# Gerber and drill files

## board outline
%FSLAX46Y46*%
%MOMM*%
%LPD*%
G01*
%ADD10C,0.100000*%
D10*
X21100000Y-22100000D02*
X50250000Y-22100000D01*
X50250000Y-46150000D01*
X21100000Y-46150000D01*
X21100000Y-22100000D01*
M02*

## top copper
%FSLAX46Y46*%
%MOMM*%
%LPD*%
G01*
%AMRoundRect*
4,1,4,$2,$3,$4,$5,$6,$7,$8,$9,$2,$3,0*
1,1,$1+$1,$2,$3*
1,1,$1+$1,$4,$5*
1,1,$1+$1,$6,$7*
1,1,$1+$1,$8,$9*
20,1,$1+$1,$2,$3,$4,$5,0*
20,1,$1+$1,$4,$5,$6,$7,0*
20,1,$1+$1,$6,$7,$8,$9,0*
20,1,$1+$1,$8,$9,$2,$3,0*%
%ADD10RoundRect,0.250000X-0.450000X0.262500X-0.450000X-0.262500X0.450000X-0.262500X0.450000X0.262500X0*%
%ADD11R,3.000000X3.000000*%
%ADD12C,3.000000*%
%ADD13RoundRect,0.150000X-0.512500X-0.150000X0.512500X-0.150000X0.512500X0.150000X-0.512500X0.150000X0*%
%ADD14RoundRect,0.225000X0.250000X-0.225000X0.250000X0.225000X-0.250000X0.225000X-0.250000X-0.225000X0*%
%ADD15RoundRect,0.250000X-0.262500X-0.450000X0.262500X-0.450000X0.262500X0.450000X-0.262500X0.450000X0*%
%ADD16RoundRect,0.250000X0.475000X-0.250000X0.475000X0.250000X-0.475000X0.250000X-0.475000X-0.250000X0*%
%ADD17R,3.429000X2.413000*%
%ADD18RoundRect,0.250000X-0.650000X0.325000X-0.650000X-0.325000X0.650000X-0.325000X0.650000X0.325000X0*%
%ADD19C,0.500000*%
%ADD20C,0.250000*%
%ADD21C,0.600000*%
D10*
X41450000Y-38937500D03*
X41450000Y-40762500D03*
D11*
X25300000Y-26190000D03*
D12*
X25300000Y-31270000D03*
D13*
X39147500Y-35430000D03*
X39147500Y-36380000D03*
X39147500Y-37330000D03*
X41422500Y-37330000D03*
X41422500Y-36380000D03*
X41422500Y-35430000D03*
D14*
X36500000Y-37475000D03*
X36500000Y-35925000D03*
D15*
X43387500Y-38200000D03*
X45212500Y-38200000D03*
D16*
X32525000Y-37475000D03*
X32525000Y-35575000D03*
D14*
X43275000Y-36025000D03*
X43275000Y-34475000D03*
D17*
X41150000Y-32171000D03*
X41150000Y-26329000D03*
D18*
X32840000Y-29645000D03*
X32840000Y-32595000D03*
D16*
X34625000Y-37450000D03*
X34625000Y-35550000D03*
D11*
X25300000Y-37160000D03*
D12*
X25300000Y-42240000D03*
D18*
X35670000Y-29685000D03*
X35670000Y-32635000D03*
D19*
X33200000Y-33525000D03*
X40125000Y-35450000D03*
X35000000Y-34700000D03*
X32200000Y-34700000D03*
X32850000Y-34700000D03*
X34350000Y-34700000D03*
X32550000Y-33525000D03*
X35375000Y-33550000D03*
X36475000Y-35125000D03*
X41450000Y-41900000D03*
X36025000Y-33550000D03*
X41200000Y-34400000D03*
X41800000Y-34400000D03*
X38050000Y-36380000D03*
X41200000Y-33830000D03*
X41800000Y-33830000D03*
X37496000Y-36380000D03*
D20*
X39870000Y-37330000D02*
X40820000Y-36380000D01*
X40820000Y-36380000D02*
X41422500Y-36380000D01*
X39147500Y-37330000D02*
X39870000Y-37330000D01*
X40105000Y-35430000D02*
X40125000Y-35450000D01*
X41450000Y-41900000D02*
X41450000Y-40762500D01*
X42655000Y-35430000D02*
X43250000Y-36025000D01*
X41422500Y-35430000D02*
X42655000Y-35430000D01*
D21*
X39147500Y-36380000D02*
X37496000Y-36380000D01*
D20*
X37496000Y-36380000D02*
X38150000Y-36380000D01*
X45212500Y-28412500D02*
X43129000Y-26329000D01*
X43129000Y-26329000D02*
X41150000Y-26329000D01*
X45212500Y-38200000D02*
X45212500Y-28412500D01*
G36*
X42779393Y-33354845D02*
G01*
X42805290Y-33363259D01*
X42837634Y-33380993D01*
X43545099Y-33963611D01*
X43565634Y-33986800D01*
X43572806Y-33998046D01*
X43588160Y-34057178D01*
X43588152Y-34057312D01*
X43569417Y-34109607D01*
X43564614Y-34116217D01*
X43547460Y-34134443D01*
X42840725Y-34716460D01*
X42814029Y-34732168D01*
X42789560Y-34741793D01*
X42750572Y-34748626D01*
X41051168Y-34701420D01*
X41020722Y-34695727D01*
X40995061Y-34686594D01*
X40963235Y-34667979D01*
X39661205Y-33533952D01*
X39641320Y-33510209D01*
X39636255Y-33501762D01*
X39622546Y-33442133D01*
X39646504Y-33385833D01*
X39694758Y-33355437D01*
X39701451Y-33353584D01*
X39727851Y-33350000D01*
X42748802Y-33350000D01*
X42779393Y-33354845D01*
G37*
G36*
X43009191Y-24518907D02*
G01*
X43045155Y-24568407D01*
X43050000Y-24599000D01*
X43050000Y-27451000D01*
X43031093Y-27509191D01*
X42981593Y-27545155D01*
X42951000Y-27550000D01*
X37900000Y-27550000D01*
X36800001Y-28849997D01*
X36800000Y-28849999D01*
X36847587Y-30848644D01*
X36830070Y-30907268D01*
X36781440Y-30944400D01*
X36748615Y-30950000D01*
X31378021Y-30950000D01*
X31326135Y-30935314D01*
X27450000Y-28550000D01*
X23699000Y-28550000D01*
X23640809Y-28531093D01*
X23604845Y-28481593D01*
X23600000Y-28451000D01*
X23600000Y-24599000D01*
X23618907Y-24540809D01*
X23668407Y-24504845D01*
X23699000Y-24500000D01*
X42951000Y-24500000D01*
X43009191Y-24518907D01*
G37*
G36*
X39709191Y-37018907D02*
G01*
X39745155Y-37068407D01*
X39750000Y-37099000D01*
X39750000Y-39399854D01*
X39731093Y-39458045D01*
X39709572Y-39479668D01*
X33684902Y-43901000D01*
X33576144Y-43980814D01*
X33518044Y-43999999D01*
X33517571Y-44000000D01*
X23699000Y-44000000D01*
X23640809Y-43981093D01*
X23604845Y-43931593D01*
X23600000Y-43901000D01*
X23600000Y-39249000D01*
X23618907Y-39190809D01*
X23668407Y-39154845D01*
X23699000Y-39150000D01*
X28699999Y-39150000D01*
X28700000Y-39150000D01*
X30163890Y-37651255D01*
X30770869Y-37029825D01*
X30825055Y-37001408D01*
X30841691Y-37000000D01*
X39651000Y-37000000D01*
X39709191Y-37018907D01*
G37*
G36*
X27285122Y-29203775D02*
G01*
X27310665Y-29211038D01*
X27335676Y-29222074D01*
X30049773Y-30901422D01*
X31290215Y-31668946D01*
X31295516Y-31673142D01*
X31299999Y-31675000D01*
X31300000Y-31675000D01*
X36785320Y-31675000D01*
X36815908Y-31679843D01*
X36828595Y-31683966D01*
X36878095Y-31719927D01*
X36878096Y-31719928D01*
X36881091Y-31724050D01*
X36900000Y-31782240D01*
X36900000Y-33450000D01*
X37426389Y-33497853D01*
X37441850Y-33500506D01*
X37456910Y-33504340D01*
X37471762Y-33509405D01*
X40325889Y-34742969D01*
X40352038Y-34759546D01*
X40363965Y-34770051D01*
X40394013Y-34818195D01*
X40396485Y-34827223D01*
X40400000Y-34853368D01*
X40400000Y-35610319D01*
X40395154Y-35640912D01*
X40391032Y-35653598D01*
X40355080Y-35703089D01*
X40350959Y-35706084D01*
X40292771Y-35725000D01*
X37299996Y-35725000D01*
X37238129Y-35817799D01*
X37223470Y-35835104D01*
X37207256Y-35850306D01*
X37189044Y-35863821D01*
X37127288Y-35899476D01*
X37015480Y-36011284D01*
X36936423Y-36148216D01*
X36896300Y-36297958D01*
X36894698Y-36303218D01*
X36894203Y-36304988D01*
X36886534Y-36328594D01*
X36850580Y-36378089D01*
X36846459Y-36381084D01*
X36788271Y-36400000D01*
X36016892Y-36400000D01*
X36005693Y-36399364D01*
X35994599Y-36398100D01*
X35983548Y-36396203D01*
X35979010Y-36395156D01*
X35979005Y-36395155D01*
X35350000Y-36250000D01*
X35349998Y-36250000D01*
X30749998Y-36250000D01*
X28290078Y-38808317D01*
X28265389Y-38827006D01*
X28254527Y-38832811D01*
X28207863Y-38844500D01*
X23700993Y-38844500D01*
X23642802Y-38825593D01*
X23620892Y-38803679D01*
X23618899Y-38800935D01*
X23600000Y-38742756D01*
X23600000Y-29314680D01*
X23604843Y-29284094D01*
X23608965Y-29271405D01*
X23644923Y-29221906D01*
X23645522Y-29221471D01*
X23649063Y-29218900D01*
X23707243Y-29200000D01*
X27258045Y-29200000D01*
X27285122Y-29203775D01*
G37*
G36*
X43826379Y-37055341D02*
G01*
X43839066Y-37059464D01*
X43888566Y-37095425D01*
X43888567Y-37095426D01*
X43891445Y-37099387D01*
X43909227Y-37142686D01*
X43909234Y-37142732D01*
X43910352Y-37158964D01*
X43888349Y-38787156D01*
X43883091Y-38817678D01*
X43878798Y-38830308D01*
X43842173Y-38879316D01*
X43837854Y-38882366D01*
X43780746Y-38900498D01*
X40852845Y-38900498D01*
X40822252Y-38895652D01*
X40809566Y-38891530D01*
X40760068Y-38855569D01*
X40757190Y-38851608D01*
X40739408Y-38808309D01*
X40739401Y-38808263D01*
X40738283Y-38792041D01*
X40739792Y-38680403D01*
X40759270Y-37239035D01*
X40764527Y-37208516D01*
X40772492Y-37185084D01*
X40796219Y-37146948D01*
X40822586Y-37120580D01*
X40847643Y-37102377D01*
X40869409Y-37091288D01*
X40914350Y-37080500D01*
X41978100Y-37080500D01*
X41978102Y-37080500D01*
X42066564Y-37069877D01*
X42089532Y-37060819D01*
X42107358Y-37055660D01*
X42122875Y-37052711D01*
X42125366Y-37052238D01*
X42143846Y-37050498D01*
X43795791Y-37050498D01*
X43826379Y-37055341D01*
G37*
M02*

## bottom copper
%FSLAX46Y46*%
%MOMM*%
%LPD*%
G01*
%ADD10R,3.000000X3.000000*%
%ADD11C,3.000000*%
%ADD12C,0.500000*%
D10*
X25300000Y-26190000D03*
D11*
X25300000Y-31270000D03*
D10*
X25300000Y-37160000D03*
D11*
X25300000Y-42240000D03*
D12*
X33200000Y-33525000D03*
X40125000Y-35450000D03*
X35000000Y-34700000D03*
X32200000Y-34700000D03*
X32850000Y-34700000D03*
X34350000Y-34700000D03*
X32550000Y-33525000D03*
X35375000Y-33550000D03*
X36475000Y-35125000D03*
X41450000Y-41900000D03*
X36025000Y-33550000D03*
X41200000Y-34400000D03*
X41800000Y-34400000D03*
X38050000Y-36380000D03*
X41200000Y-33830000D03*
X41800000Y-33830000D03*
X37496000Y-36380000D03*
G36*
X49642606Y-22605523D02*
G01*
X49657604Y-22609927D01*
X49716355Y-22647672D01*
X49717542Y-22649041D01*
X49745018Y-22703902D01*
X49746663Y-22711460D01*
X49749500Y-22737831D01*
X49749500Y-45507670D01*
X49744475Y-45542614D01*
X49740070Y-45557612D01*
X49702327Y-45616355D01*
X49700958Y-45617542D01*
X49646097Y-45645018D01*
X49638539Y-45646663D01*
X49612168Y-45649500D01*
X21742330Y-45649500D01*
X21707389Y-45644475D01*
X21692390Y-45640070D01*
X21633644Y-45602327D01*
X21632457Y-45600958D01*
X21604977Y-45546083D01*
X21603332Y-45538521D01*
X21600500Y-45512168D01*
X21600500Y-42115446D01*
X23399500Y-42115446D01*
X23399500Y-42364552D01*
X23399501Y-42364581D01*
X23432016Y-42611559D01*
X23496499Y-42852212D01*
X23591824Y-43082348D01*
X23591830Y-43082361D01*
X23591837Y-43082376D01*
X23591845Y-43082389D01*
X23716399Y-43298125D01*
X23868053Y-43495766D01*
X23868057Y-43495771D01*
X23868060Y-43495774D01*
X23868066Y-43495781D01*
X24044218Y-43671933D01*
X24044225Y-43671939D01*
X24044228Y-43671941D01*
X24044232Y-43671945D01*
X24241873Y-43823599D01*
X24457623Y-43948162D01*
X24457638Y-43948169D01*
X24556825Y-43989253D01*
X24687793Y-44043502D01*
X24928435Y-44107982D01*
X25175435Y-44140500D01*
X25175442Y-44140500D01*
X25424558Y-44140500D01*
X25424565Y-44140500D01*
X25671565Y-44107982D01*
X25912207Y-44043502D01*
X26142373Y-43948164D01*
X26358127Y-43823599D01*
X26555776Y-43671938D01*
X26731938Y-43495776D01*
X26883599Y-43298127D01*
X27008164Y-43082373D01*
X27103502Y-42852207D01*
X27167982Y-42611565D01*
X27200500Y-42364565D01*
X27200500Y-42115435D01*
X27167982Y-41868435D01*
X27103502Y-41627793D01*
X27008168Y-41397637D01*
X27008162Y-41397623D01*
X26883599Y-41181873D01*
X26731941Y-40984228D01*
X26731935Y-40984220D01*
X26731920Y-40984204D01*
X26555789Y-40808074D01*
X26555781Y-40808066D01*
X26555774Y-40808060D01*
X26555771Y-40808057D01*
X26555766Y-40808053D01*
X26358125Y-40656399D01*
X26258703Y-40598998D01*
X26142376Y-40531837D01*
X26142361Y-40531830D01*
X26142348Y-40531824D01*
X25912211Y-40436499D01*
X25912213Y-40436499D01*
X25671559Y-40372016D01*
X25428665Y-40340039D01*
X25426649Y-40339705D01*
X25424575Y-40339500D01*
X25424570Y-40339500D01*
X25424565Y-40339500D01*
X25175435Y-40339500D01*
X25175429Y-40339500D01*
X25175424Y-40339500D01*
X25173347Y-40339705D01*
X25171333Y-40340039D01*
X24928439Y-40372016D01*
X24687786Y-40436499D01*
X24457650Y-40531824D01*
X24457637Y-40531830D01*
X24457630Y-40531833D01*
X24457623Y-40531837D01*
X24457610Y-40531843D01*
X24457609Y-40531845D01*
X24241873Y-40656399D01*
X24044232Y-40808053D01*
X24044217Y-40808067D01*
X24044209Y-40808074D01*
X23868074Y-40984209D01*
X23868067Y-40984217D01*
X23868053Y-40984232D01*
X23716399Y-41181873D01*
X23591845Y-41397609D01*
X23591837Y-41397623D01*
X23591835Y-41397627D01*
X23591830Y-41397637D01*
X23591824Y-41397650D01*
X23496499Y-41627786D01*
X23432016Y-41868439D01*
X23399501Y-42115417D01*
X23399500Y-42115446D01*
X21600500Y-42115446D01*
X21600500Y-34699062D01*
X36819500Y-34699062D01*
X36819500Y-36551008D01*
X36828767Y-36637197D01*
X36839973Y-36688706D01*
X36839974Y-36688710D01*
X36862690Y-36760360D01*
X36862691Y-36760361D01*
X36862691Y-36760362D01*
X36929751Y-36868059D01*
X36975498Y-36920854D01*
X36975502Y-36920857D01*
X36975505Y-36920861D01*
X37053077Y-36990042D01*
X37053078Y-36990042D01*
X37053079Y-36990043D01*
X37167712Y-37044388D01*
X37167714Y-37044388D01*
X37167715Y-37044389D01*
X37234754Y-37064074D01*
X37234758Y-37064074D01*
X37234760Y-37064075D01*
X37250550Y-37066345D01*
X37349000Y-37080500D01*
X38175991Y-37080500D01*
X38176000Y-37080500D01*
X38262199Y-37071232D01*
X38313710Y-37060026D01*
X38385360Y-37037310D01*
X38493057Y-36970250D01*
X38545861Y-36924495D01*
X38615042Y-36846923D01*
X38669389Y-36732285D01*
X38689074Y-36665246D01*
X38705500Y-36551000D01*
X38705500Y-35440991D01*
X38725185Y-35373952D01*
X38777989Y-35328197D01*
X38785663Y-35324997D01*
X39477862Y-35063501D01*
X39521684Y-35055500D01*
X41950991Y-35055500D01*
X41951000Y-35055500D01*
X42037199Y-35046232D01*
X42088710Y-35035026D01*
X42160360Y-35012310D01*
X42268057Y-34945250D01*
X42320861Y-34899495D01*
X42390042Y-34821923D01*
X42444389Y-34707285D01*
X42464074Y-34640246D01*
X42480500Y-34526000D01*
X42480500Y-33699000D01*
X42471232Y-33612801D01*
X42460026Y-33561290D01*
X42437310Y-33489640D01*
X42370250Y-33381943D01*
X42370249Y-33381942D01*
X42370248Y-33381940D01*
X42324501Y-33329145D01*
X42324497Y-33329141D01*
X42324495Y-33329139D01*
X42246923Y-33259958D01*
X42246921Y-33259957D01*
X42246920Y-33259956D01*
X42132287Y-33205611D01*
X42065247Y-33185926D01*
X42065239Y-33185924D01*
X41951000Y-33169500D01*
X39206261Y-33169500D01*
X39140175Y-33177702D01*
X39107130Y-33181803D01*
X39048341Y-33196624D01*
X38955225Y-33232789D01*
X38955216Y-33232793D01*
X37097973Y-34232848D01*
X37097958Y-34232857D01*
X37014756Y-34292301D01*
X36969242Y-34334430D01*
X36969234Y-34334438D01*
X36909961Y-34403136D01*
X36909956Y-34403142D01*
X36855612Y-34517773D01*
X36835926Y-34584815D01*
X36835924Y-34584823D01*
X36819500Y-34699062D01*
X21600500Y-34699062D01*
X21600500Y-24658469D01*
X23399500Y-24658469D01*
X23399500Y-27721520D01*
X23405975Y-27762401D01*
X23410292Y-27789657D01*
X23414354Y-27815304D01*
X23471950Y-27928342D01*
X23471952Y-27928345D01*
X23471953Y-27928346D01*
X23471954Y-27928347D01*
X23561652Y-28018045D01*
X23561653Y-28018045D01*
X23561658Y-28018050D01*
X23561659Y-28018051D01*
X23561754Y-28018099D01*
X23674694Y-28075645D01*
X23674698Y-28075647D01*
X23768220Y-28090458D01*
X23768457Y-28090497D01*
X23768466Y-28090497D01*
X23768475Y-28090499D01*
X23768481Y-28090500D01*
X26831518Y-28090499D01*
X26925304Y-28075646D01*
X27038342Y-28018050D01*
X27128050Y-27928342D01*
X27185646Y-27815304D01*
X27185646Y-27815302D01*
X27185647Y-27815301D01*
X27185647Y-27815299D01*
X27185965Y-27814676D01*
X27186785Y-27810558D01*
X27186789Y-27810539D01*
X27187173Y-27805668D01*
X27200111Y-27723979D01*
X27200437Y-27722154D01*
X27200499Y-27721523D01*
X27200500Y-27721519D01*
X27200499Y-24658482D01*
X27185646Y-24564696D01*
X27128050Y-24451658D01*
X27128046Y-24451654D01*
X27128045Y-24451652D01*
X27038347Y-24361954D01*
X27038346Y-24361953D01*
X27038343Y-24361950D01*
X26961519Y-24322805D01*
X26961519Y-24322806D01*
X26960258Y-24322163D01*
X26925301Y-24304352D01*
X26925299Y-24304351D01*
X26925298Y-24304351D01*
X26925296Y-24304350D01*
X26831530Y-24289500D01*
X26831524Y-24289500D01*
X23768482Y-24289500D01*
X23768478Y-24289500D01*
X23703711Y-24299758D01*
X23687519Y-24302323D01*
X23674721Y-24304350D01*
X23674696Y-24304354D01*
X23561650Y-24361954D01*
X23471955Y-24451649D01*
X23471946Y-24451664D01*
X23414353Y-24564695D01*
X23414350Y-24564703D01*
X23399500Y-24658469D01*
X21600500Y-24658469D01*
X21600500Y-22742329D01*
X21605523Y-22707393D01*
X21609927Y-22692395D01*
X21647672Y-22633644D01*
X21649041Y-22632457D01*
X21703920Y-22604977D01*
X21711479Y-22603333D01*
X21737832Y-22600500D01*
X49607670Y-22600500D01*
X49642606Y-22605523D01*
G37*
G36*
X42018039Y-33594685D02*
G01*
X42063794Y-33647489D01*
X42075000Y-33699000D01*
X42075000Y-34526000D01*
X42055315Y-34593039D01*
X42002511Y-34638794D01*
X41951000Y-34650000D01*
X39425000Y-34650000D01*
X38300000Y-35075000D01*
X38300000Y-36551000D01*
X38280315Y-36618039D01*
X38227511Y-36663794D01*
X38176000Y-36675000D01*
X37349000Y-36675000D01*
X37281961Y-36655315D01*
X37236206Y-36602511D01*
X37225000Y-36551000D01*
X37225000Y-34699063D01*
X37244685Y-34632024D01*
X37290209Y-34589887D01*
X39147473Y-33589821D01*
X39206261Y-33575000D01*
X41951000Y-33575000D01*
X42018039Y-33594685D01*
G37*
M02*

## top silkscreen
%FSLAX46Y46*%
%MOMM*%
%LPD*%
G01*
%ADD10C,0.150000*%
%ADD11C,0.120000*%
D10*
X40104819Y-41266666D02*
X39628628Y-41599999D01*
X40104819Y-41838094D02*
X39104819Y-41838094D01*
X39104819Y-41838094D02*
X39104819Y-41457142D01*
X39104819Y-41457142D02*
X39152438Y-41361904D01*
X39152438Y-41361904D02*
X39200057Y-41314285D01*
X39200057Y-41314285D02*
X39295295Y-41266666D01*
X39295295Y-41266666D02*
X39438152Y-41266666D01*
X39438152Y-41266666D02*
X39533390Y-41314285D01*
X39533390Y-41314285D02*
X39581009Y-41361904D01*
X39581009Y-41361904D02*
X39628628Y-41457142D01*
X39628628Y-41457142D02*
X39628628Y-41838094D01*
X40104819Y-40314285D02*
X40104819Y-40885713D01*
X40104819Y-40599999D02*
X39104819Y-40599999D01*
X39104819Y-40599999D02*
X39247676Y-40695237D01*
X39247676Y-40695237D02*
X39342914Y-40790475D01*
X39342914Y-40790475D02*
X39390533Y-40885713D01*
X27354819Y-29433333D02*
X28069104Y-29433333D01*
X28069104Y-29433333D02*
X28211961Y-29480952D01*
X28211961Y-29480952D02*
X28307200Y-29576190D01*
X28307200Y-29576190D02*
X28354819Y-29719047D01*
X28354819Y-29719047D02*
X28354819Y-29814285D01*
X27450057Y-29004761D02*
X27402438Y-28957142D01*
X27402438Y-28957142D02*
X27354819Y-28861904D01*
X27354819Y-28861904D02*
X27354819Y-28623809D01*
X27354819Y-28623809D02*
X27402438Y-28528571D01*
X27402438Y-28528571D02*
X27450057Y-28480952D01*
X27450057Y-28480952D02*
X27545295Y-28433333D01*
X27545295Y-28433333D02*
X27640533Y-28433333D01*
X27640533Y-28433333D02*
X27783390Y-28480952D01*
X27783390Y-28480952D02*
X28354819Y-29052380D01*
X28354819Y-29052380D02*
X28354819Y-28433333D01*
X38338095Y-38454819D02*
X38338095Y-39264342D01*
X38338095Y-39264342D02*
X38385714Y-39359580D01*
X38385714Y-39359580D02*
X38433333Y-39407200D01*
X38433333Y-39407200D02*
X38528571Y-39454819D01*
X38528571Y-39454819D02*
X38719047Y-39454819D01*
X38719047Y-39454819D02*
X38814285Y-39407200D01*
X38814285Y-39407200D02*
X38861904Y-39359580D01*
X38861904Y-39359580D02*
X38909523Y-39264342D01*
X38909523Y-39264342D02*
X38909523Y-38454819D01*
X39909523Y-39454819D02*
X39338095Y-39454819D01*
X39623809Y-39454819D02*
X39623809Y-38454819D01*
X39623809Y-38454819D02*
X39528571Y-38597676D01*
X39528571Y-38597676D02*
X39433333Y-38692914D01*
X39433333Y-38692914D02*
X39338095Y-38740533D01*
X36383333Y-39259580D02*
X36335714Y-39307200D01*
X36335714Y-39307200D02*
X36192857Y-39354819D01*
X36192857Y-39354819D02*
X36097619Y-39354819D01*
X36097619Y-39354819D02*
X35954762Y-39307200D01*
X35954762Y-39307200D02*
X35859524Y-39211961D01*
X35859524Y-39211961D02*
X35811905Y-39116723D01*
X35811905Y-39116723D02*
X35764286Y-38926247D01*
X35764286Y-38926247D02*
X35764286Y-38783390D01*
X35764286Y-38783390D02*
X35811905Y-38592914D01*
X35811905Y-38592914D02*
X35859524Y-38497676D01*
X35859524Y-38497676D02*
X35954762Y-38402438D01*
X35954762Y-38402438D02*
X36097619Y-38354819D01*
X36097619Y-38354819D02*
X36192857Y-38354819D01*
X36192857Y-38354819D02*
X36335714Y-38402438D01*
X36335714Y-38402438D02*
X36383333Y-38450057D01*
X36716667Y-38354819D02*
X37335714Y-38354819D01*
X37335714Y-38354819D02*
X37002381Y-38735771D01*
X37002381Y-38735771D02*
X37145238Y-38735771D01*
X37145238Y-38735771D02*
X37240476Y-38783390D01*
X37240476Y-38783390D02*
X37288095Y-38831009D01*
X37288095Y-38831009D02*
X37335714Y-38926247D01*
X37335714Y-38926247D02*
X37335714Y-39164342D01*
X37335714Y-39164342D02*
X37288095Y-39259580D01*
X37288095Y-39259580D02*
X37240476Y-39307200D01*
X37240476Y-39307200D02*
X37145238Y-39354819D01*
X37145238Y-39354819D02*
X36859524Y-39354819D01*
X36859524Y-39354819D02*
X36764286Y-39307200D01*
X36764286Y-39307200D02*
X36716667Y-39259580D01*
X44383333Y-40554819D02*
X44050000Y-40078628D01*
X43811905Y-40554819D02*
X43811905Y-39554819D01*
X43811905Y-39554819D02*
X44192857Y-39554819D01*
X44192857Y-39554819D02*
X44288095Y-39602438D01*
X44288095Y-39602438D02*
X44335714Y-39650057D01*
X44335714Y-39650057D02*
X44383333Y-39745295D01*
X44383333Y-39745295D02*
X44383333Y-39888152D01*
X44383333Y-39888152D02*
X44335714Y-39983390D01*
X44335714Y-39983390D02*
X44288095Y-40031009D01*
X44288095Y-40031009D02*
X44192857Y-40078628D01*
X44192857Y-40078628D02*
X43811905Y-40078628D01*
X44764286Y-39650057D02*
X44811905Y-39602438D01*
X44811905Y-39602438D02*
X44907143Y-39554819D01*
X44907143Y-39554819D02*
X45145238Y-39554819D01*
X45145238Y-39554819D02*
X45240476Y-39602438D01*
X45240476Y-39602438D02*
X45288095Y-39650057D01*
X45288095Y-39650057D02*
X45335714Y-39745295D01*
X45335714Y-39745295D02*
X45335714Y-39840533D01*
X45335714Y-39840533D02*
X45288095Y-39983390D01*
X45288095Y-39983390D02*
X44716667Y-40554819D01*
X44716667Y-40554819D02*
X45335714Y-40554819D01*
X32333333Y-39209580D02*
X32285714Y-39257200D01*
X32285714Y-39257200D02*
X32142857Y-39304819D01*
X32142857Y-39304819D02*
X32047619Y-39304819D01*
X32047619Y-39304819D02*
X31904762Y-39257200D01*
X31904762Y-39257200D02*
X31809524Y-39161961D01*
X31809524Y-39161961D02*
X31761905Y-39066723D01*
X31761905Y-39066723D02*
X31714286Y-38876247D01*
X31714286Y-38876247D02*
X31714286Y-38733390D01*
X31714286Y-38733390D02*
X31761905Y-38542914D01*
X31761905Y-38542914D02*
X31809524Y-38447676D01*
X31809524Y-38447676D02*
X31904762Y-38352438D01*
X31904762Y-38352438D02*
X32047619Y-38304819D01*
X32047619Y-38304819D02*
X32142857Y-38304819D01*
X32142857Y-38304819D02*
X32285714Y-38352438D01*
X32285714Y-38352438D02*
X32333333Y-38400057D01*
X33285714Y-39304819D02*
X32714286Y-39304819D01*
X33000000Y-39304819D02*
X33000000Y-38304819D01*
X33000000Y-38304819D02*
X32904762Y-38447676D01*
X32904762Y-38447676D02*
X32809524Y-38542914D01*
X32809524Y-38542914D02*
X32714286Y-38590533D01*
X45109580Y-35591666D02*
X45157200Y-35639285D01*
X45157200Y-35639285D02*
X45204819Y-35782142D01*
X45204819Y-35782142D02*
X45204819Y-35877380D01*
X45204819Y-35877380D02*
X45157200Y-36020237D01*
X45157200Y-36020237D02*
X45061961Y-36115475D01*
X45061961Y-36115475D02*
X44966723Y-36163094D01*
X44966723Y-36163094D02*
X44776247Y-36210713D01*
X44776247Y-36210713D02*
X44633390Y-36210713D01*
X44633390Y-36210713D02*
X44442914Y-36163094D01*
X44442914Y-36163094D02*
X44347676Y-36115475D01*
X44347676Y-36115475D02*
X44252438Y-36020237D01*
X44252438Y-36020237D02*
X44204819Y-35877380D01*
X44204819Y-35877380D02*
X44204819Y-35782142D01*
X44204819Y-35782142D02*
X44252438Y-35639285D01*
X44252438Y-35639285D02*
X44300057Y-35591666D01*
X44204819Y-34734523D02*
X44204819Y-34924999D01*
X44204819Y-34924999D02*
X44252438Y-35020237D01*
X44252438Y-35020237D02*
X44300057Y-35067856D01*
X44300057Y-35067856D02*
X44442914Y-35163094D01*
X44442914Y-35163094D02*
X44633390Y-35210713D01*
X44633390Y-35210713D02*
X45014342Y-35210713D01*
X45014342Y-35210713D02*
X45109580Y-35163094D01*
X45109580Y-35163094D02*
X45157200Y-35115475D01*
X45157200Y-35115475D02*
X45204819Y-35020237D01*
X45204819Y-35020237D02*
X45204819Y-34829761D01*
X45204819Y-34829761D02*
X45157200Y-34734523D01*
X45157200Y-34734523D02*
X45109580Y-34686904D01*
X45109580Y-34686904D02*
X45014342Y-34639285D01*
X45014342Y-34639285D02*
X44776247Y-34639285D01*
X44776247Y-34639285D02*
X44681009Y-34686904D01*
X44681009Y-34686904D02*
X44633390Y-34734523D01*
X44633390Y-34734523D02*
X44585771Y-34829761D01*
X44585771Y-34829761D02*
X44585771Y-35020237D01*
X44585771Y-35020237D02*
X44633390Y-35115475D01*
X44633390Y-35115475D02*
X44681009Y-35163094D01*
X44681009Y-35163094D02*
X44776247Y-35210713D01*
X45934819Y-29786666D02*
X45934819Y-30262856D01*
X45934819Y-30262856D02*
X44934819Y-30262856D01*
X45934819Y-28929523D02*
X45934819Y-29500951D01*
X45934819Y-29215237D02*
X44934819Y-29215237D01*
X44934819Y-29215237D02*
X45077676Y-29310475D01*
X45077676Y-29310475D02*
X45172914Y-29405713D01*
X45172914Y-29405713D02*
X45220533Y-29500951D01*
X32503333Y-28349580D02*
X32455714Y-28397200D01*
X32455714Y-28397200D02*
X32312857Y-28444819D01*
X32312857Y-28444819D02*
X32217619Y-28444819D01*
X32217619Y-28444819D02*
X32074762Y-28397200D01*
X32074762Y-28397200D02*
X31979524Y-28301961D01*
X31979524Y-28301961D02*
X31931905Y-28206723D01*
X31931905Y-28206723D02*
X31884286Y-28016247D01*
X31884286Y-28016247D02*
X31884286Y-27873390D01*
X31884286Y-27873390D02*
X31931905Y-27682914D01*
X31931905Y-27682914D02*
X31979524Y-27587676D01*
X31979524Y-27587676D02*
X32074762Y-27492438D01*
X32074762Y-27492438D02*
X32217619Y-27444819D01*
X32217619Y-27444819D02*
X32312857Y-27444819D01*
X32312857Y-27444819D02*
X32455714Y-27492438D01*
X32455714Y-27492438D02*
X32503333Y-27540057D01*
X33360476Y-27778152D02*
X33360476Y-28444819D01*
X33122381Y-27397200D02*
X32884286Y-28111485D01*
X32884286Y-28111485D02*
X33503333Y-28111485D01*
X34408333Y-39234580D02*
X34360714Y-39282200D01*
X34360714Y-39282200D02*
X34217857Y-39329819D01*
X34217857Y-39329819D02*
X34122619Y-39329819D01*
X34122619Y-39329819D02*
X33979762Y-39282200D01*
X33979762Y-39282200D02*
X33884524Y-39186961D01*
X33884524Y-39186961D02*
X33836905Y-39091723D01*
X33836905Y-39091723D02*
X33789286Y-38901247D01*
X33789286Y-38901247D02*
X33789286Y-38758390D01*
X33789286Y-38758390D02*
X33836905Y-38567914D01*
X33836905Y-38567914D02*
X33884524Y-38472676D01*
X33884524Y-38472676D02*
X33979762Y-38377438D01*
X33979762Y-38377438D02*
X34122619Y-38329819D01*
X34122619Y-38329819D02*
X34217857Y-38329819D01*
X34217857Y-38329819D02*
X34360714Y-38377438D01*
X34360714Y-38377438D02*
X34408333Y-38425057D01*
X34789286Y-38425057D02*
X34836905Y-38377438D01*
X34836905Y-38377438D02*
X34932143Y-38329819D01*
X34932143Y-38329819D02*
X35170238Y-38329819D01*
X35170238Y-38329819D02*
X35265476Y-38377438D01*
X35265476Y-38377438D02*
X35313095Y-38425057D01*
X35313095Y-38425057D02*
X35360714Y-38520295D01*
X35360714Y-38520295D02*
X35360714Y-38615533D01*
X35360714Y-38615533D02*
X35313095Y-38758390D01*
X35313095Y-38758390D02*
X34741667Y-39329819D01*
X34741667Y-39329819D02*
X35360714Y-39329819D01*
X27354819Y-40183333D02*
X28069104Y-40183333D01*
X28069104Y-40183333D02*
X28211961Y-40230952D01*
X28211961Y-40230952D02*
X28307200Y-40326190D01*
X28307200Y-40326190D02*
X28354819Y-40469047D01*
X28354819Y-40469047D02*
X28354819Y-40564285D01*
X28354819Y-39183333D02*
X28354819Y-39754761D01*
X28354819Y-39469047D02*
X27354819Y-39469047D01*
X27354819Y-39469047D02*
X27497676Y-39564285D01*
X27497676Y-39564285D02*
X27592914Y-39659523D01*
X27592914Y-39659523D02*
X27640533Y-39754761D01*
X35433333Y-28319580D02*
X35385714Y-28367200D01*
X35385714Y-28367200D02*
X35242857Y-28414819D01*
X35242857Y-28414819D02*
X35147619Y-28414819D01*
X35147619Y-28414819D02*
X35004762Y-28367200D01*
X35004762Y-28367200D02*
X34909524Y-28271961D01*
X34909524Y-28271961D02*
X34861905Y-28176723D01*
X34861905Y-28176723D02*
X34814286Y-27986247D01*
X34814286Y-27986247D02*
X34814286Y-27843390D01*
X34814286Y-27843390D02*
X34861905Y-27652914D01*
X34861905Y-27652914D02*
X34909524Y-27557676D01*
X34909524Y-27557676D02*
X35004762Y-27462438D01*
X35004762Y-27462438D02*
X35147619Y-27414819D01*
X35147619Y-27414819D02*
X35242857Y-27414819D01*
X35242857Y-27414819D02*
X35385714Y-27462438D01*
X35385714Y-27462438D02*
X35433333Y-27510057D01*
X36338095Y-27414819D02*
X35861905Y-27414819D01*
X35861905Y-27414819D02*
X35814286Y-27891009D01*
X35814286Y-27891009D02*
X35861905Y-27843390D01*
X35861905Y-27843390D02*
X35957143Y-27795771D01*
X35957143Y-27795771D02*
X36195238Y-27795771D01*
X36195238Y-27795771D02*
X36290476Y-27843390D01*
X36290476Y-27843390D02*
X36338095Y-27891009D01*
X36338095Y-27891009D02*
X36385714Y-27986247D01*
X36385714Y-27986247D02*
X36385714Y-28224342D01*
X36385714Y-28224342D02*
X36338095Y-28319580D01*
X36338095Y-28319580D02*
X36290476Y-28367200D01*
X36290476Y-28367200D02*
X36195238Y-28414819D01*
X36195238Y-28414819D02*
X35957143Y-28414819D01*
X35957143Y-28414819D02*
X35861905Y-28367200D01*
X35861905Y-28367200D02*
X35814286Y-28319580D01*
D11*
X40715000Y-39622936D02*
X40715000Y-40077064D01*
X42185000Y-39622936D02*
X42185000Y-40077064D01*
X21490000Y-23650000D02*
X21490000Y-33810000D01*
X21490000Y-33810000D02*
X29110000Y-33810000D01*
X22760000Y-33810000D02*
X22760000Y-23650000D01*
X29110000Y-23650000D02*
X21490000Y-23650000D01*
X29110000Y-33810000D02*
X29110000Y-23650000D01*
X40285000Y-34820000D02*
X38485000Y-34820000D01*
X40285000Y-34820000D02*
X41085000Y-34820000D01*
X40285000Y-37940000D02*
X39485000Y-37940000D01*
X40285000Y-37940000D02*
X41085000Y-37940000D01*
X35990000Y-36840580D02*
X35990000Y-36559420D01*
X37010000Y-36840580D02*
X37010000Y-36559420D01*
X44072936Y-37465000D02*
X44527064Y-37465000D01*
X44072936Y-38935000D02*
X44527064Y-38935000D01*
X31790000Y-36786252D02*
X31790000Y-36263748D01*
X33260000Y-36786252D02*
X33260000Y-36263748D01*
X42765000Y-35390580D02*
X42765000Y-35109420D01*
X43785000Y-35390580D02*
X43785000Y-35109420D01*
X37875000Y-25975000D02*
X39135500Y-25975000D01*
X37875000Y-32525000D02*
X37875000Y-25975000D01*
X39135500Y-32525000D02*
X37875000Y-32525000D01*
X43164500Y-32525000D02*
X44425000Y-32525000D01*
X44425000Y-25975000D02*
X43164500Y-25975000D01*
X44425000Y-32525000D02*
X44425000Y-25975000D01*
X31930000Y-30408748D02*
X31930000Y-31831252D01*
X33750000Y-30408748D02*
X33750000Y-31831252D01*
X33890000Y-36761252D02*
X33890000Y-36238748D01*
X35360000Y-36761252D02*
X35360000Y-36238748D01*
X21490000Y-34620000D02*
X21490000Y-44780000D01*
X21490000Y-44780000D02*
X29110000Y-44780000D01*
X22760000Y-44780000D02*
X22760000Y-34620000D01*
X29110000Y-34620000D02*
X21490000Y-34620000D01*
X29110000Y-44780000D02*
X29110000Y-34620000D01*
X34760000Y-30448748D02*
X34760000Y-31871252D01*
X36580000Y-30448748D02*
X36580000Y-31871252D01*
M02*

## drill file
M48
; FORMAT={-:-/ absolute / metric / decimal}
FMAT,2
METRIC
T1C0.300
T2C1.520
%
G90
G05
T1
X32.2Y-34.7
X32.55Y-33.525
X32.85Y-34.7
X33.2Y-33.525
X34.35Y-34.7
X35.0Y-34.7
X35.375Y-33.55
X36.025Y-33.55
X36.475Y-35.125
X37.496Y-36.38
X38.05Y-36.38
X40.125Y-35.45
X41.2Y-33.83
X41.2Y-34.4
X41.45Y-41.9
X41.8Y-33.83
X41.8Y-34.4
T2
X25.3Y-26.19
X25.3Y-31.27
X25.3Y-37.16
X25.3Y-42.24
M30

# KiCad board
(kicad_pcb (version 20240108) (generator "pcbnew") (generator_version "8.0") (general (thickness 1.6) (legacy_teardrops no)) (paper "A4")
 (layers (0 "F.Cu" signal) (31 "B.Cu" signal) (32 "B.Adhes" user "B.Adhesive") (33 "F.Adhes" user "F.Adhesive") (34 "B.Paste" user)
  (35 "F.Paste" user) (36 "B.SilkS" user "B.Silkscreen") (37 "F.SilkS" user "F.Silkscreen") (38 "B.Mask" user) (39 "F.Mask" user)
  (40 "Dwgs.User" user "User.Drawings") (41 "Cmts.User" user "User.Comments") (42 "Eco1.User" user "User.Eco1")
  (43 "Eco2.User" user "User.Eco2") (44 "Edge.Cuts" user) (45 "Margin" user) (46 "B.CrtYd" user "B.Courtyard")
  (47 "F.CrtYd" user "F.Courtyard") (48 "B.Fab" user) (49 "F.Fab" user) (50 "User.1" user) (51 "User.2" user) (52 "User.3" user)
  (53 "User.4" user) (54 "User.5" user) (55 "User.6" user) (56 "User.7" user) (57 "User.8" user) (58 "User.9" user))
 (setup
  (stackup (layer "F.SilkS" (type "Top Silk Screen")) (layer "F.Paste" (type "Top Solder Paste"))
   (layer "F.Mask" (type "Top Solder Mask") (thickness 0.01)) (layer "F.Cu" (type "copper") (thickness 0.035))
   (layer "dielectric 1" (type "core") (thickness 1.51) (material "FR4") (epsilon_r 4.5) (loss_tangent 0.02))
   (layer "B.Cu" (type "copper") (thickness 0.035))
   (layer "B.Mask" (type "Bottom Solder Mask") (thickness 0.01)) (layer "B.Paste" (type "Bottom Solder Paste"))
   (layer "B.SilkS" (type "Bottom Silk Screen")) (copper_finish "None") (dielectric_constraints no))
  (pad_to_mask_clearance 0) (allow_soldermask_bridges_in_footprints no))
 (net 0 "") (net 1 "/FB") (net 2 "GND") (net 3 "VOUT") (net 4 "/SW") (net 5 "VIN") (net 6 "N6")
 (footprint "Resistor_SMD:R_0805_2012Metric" (layer "F.Cu") (at 41.45 39.85 -90)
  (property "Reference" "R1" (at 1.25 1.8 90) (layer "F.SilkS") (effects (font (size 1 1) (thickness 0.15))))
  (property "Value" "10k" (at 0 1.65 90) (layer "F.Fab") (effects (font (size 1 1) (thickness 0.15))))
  (fp_line (start -0.227064 0.735) (end 0.227064 0.735) (stroke (width 0.12) (type solid)) (layer "F.SilkS"))
  (fp_line (start -0.227064 -0.735) (end 0.227064 -0.735) (stroke (width 0.12) (type solid)) (layer "F.SilkS"))
  (pad "1" smd roundrect (at -0.9125 0 270) (size 1.025 1.4) (layers "F.Cu" "F.Paste" "F.Mask") (roundrect_rratio 0.243902) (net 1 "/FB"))
  (pad "2" smd roundrect (at 0.9125 0 270) (size 1.025 1.4) (layers "F.Cu" "F.Paste" "F.Mask") (roundrect_rratio 0.243902) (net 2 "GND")))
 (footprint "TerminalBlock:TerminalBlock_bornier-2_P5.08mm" (layer "F.Cu") (at 25.3 26.19 -90)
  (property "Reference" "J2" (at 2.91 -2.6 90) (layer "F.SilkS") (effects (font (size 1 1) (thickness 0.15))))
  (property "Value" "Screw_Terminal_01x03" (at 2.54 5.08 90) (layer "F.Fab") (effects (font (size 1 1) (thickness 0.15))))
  (fp_line (start -2.54 3.81) (end 7.62 3.81) (stroke (width 0.12) (type solid)) (layer "F.SilkS"))
  (fp_line (start 7.62 3.81) (end 7.62 -3.81) (stroke (width 0.12) (type solid)) (layer "F.SilkS"))
  (fp_line (start 7.62 2.54) (end -2.54 2.54) (stroke (width 0.12) (type solid)) (layer "F.SilkS"))
  (fp_line (start -2.54 -3.81) (end -2.54 3.81) (stroke (width 0.12) (type solid)) (layer "F.SilkS"))
  (fp_line (start 7.62 -3.81) (end -2.54 -3.81) (stroke (width 0.12) (type solid)) (layer "F.SilkS"))
  (pad "1" thru_hole rect (at 0 0 270) (size 3 3) (drill 1.52) (layers "*.Cu" "*.Mask") (remove_unused_layers no) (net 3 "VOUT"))
  (pad "2" thru_hole circle (at 5.08 0 270) (size 3 3) (drill 1.52) (layers "*.Cu" "*.Mask") (remove_unused_layers no) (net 2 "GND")))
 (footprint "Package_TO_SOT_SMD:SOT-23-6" (layer "F.Cu") (at 40.285 36.38)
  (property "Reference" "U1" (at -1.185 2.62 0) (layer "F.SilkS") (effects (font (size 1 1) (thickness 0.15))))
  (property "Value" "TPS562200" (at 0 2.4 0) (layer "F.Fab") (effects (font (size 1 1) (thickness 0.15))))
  (fp_line (start 0 -1.56) (end -1.8 -1.56) (stroke (width 0.12) (type solid)) (layer "F.SilkS"))
  (fp_line (start 0 -1.56) (end 0.8 -1.56) (stroke (width 0.12) (type solid)) (layer "F.SilkS"))
  (fp_line (start 0 1.56) (end -0.8 1.56) (stroke (width 0.12) (type solid)) (layer "F.SilkS"))
  (fp_line (start 0 1.56) (end 0.8 1.56) (stroke (width 0.12) (type solid)) (layer "F.SilkS"))
  (pad "1" smd roundrect (at -1.1375 -0.95) (size 1.325 0.6) (layers "F.Cu" "F.Paste" "F.Mask") (roundrect_rratio 0.25) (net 2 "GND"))
  (pad "2" smd roundrect (at -1.1375 0) (size 1.325 0.6) (layers "F.Cu" "F.Paste" "F.Mask") (roundrect_rratio 0.25) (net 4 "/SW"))
  (pad "3" smd roundrect (at -1.1375 0.95) (size 1.325 0.6) (layers "F.Cu" "F.Paste" "F.Mask") (roundrect_rratio 0.25) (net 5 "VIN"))
  (pad "4" smd roundrect (at 1.1375 0.95) (size 1.325 0.6) (layers "F.Cu" "F.Paste" "F.Mask") (roundrect_rratio 0.25) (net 1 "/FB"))
  (pad "5" smd roundrect (at 1.1375 0) (size 1.325 0.6) (layers "F.Cu" "F.Paste" "F.Mask") (roundrect_rratio 0.25) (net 5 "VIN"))
  (pad "6" smd roundrect (at 1.1375 -0.95) (size 1.325 0.6) (layers "F.Cu" "F.Paste" "F.Mask") (roundrect_rratio 0.25) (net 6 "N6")))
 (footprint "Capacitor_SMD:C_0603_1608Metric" (layer "F.Cu") (at 36.5 36.7 90)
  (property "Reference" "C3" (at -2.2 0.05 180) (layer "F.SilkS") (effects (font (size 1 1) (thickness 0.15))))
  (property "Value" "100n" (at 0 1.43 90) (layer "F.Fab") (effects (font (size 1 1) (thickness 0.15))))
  (fp_line (start -0.14058 -0.51) (end 0.14058 -0.51) (stroke (width 0.12) (type solid)) (layer "F.SilkS"))
  (fp_line (start -0.14058 0.51) (end 0.14058 0.51) (stroke (width 0.12) (type solid)) (layer "F.SilkS"))
  (pad "1" smd roundrect (at -0.775 0 90) (size 0.9 0.95) (layers "F.Cu" "F.Paste" "F.Mask") (roundrect_rratio 0.25) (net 5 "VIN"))
  (pad "2" smd roundrect (at 0.775 0 90) (size 0.9 0.95) (layers "F.Cu" "F.Paste" "F.Mask") (roundrect_rratio 0.25) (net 2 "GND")))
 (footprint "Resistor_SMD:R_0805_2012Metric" (layer "F.Cu") (at 44.3 38.2)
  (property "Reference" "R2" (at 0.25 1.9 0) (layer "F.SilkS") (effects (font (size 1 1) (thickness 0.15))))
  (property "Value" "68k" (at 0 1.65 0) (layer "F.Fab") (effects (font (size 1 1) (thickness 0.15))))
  (fp_line (start -0.227064 -0.735) (end 0.227064 -0.735) (stroke (width 0.12) (type solid)) (layer "F.SilkS"))
  (fp_line (start -0.227064 0.735) (end 0.227064 0.735) (stroke (width 0.12) (type solid)) (layer "F.SilkS"))
  (pad "1" smd roundrect (at -0.9125 0) (size 1.025 1.4) (layers "F.Cu" "F.Paste" "F.Mask") (roundrect_rratio 0.243902) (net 1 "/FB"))
  (pad "2" smd roundrect (at 0.9125 0) (size 1.025 1.4) (layers "F.Cu" "F.Paste" "F.Mask") (roundrect_rratio 0.243902) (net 3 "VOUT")))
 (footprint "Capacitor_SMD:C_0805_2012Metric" (layer "F.Cu") (at 32.525 36.525 90)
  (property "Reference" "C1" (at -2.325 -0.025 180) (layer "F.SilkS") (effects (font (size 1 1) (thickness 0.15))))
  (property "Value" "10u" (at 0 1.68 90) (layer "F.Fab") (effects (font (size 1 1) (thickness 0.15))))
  (fp_line (start -0.261252 -0.735) (end 0.261252 -0.735) (stroke (width 0.12) (type solid)) (layer "F.SilkS"))
  (fp_line (start -0.261252 0.735) (end 0.261252 0.735) (stroke (width 0.12) (type solid)) (layer "F.SilkS"))
  (pad "1" smd roundrect (at -0.95 0 90) (size 1 1.45) (layers "F.Cu" "F.Paste" "F.Mask") (roundrect_rratio 0.25) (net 5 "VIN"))
  (pad "2" smd roundrect (at 0.95 0 90) (size 1 1.45) (layers "F.Cu" "F.Paste" "F.Mask") (roundrect_rratio 0.25) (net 2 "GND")))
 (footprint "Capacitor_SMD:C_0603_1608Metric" (layer "F.Cu") (at 43.275 35.25 90)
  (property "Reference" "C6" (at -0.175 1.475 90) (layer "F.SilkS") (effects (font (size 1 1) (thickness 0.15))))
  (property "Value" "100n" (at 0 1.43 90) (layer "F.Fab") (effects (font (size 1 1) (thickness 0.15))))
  (fp_line (start -0.14058 -0.51) (end 0.14058 -0.51) (stroke (width 0.12) (type solid)) (layer "F.SilkS"))
  (fp_line (start -0.14058 0.51) (end 0.14058 0.51) (stroke (width 0.12) (type solid)) (layer "F.SilkS"))
  (pad "1" smd roundrect (at -0.775 0 90) (size 0.9 0.95) (layers "F.Cu" "F.Paste" "F.Mask") (roundrect_rratio 0.25) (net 6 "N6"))
  (pad "2" smd roundrect (at 0.775 0 90) (size 0.9 0.95) (layers "F.Cu" "F.Paste" "F.Mask") (roundrect_rratio 0.25) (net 4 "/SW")))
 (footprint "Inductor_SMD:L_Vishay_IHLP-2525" (layer "F.Cu") (at 41.15 29.25 90)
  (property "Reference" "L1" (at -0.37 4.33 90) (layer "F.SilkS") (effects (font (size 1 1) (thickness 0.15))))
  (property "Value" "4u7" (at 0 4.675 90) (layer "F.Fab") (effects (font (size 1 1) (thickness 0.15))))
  (fp_line (start 3.275 -3.275) (end 3.275 -2.0145) (stroke (width 0.12) (type solid)) (layer "F.SilkS"))
  (fp_line (start -3.275 -3.275) (end 3.275 -3.275) (stroke (width 0.12) (type solid)) (layer "F.SilkS"))
  (fp_line (start -3.275 -2.0145) (end -3.275 -3.275) (stroke (width 0.12) (type solid)) (layer "F.SilkS"))
  (fp_line (start -3.275 2.0145) (end -3.275 3.275) (stroke (width 0.12) (type solid)) (layer "F.SilkS"))
  (fp_line (start 3.275 3.275) (end 3.275 2.0145) (stroke (width 0.12) (type solid)) (layer "F.SilkS"))
  (fp_line (start -3.275 3.275) (end 3.275 3.275) (stroke (width 0.12) (type solid)) (layer "F.SilkS"))
  (pad "1" smd rect (at -2.921 0 90) (size 2.413 3.429) (layers "F.Cu" "F.Paste" "F.Mask") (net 4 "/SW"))
  (pad "2" smd rect (at 2.921 0 90) (size 2.413 3.429) (layers "F.Cu" "F.Paste" "F.Mask") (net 3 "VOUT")))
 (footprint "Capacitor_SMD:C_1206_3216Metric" (layer "F.Cu") (at 32.84 31.12 -90)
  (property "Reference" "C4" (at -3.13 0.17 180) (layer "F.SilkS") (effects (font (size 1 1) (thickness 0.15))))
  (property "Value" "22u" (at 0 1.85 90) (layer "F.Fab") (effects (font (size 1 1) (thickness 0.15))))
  (fp_line (start -0.711252 0.91) (end 0.711252 0.91) (stroke (width 0.12) (type solid)) (layer "F.SilkS"))
  (fp_line (start -0.711252 -0.91) (end 0.711252 -0.91) (stroke (width 0.12) (type solid)) (layer "F.SilkS"))
  (pad "1" smd roundrect (at -1.475 0 270) (size 1.15 1.8) (layers "F.Cu" "F.Paste" "F.Mask") (roundrect_rratio 0.217391) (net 3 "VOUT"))
  (pad "2" smd roundrect (at 1.475 0 270) (size 1.15 1.8) (layers "F.Cu" "F.Paste" "F.Mask") (roundrect_rratio 0.217391) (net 2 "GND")))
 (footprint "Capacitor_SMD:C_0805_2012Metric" (layer "F.Cu") (at 34.625 36.5 90)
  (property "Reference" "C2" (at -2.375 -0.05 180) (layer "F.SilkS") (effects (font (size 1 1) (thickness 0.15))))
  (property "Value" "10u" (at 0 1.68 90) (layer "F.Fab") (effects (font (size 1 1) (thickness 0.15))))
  (fp_line (start -0.261252 -0.735) (end 0.261252 -0.735) (stroke (width 0.12) (type solid)) (layer "F.SilkS"))
  (fp_line (start -0.261252 0.735) (end 0.261252 0.735) (stroke (width 0.12) (type solid)) (layer "F.SilkS"))
  (pad "1" smd roundrect (at -0.95 0 90) (size 1 1.45) (layers "F.Cu" "F.Paste" "F.Mask") (roundrect_rratio 0.25) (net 5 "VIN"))
  (pad "2" smd roundrect (at 0.95 0 90) (size 1 1.45) (layers "F.Cu" "F.Paste" "F.Mask") (roundrect_rratio 0.25) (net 2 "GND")))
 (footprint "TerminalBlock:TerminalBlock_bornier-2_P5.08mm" (layer "F.Cu") (at 25.3 37.16 -90)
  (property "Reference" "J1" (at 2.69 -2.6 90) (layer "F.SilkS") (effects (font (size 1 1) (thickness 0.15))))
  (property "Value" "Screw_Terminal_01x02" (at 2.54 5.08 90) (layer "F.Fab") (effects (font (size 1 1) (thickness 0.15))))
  (fp_line (start -2.54 3.81) (end 7.62 3.81) (stroke (width 0.12) (type solid)) (layer "F.SilkS"))
  (fp_line (start 7.62 3.81) (end 7.62 -3.81) (stroke (width 0.12) (type solid)) (layer "F.SilkS"))
  (fp_line (start 7.62 2.54) (end -2.54 2.54) (stroke (width 0.12) (type solid)) (layer "F.SilkS"))
  (fp_line (start -2.54 -3.81) (end -2.54 3.81) (stroke (width 0.12) (type solid)) (layer "F.SilkS"))
  (fp_line (start 7.62 -3.81) (end -2.54 -3.81) (stroke (width 0.12) (type solid)) (layer "F.SilkS"))
  (pad "1" thru_hole rect (at 0 0 270) (size 3 3) (drill 1.52) (layers "*.Cu" "*.Mask") (remove_unused_layers no) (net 2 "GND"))
  (pad "2" thru_hole circle (at 5.08 0 270) (size 3 3) (drill 1.52) (layers "*.Cu" "*.Mask") (remove_unused_layers no) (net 5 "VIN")))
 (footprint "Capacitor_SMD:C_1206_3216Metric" (layer "F.Cu") (at 35.67 31.16 -90)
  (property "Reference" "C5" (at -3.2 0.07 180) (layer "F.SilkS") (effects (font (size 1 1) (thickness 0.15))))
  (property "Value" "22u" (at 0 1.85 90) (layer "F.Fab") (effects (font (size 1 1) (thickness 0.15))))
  (fp_line (start -0.711252 0.91) (end 0.711252 0.91) (stroke (width 0.12) (type solid)) (layer "F.SilkS"))
  (fp_line (start -0.711252 -0.91) (end 0.711252 -0.91) (stroke (width 0.12) (type solid)) (layer "F.SilkS"))
  (pad "1" smd roundrect (at -1.475 0 270) (size 1.15 1.8) (layers "F.Cu" "F.Paste" "F.Mask") (roundrect_rratio 0.217391) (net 3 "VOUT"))
  (pad "2" smd roundrect (at 1.475 0 270) (size 1.15 1.8) (layers "F.Cu" "F.Paste" "F.Mask") (roundrect_rratio 0.217391) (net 2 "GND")))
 (gr_rect (start 21.1 22.1) (end 50.25 46.15) (stroke (width 0.1) (type default)) (fill none) (layer "Edge.Cuts"))
 (segment (start 39.87 37.33) (end 40.82 36.38) (width 0.25) (layer "F.Cu") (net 5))
 (segment (start 40.82 36.38) (end 41.4225 36.38) (width 0.25) (layer "F.Cu") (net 5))
 (segment (start 39.1475 37.33) (end 39.87 37.33) (width 0.25) (layer "F.Cu") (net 5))
 (segment (start 40.105 35.43) (end 40.125 35.45) (width 0.25) (layer "F.Cu") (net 2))
 (segment (start 41.45 41.9) (end 41.45 40.7625) (width 0.25) (layer "F.Cu") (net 2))
 (via (at 33.2 33.525) (size 0.5) (drill 0.3) (layers "F.Cu" "B.Cu") (free yes) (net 2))
 (via (at 40.125 35.45) (size 0.5) (drill 0.3) (layers "F.Cu" "B.Cu") (free yes) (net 2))
 (via (at 35 34.7) (size 0.5) (drill 0.3) (layers "F.Cu" "B.Cu") (free yes) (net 2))
 (via (at 32.2 34.7) (size 0.5) (drill 0.3) (layers "F.Cu" "B.Cu") (free yes) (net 2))
 (via (at 32.85 34.7) (size 0.5) (drill 0.3) (layers "F.Cu" "B.Cu") (free yes) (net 2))
 (via (at 34.35 34.7) (size 0.5) (drill 0.3) (layers "F.Cu" "B.Cu") (free yes) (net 2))
 (via (at 32.55 33.525) (size 0.5) (drill 0.3) (layers "F.Cu" "B.Cu") (free yes) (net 2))
 (via (at 35.375 33.55) (size 0.5) (drill 0.3) (layers "F.Cu" "B.Cu") (free yes) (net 2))
 (via (at 36.475 35.125) (size 0.5) (drill 0.3) (layers "F.Cu" "B.Cu") (free yes) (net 2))
 (via (at 41.45 41.9) (size 0.5) (drill 0.3) (layers "F.Cu" "B.Cu") (free yes) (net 2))
 (via (at 36.025 33.55) (size 0.5) (drill 0.3) (layers "F.Cu" "B.Cu") (free yes) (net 2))
 (segment (start 42.655 35.43) (end 43.25 36.025) (width 0.25) (layer "F.Cu") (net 6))
 (segment (start 41.4225 35.43) (end 42.655 35.43) (width 0.25) (layer "F.Cu") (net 6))
 (segment (start 39.1475 36.38) (end 37.496 36.38) (width 0.6) (layer "F.Cu") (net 4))
 (segment (start 37.496 36.38) (end 38.15 36.38) (width 0.25) (layer "F.Cu") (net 4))
 (via (at 41.2 34.4) (size 0.5) (drill 0.3) (layers "F.Cu" "B.Cu") (free yes) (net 4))
 (via (at 41.8 34.4) (size 0.5) (drill 0.3) (layers "F.Cu" "B.Cu") (free yes) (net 4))
 (via (at 38.05 36.38) (size 0.5) (drill 0.3) (layers "F.Cu" "B.Cu") (free yes) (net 4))
 (via (at 41.2 33.83) (size 0.5) (drill 0.3) (layers "F.Cu" "B.Cu") (free yes) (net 4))
 (via (at 41.8 33.83) (size 0.5) (drill 0.3) (layers "F.Cu" "B.Cu") (free yes) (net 4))
 (via (at 37.496 36.38) (size 0.5) (drill 0.3) (layers "F.Cu" "B.Cu") (free yes) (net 4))
 (segment (start 45.2125 28.4125) (end 43.129 26.329) (width 0.25) (layer "F.Cu") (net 3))
 (segment (start 43.129 26.329) (end 41.15 26.329) (width 0.25) (layer "F.Cu") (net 3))
 (segment (start 45.2125 38.2) (end 45.2125 28.4125) (width 0.25) (layer "F.Cu") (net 3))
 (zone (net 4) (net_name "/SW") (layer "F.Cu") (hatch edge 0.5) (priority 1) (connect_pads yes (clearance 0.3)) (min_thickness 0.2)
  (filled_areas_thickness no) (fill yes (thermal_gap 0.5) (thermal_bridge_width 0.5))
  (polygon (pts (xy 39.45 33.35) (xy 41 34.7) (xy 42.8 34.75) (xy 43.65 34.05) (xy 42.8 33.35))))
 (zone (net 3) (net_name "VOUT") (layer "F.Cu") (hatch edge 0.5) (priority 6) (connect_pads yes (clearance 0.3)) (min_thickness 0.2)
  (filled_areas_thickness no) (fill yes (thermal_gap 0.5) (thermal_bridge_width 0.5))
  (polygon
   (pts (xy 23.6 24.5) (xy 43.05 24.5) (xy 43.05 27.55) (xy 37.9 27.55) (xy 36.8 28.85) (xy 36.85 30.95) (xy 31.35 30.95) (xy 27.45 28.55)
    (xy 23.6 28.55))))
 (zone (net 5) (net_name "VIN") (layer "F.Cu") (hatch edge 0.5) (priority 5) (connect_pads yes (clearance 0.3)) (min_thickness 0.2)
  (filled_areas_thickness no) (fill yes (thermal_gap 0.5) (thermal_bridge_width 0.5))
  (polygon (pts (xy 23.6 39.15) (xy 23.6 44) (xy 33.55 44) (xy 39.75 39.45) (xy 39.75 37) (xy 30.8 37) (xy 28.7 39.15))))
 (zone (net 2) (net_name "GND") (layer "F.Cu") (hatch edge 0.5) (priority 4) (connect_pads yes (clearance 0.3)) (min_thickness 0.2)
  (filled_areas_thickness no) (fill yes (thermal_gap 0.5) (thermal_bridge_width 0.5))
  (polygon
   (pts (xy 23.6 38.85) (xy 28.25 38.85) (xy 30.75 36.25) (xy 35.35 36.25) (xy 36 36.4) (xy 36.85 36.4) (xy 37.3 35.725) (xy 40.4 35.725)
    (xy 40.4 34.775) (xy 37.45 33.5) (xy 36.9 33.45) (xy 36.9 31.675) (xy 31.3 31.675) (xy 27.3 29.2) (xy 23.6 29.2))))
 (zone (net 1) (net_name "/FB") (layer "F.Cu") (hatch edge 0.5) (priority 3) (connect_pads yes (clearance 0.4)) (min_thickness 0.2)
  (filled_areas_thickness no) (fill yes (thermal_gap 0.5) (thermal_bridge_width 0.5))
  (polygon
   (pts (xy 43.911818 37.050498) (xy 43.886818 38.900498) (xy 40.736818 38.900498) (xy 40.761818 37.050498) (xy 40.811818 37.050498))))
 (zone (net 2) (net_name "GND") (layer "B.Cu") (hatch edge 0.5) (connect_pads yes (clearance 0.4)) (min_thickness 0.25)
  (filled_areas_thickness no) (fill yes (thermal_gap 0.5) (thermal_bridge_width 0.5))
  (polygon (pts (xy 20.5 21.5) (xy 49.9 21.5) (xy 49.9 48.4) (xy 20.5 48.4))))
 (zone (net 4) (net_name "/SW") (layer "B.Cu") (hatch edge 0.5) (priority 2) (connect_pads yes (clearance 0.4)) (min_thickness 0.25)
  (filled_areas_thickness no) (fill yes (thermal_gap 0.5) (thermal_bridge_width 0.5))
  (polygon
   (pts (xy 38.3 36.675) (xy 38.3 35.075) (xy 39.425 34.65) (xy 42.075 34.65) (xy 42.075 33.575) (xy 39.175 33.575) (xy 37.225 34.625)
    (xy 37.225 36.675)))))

